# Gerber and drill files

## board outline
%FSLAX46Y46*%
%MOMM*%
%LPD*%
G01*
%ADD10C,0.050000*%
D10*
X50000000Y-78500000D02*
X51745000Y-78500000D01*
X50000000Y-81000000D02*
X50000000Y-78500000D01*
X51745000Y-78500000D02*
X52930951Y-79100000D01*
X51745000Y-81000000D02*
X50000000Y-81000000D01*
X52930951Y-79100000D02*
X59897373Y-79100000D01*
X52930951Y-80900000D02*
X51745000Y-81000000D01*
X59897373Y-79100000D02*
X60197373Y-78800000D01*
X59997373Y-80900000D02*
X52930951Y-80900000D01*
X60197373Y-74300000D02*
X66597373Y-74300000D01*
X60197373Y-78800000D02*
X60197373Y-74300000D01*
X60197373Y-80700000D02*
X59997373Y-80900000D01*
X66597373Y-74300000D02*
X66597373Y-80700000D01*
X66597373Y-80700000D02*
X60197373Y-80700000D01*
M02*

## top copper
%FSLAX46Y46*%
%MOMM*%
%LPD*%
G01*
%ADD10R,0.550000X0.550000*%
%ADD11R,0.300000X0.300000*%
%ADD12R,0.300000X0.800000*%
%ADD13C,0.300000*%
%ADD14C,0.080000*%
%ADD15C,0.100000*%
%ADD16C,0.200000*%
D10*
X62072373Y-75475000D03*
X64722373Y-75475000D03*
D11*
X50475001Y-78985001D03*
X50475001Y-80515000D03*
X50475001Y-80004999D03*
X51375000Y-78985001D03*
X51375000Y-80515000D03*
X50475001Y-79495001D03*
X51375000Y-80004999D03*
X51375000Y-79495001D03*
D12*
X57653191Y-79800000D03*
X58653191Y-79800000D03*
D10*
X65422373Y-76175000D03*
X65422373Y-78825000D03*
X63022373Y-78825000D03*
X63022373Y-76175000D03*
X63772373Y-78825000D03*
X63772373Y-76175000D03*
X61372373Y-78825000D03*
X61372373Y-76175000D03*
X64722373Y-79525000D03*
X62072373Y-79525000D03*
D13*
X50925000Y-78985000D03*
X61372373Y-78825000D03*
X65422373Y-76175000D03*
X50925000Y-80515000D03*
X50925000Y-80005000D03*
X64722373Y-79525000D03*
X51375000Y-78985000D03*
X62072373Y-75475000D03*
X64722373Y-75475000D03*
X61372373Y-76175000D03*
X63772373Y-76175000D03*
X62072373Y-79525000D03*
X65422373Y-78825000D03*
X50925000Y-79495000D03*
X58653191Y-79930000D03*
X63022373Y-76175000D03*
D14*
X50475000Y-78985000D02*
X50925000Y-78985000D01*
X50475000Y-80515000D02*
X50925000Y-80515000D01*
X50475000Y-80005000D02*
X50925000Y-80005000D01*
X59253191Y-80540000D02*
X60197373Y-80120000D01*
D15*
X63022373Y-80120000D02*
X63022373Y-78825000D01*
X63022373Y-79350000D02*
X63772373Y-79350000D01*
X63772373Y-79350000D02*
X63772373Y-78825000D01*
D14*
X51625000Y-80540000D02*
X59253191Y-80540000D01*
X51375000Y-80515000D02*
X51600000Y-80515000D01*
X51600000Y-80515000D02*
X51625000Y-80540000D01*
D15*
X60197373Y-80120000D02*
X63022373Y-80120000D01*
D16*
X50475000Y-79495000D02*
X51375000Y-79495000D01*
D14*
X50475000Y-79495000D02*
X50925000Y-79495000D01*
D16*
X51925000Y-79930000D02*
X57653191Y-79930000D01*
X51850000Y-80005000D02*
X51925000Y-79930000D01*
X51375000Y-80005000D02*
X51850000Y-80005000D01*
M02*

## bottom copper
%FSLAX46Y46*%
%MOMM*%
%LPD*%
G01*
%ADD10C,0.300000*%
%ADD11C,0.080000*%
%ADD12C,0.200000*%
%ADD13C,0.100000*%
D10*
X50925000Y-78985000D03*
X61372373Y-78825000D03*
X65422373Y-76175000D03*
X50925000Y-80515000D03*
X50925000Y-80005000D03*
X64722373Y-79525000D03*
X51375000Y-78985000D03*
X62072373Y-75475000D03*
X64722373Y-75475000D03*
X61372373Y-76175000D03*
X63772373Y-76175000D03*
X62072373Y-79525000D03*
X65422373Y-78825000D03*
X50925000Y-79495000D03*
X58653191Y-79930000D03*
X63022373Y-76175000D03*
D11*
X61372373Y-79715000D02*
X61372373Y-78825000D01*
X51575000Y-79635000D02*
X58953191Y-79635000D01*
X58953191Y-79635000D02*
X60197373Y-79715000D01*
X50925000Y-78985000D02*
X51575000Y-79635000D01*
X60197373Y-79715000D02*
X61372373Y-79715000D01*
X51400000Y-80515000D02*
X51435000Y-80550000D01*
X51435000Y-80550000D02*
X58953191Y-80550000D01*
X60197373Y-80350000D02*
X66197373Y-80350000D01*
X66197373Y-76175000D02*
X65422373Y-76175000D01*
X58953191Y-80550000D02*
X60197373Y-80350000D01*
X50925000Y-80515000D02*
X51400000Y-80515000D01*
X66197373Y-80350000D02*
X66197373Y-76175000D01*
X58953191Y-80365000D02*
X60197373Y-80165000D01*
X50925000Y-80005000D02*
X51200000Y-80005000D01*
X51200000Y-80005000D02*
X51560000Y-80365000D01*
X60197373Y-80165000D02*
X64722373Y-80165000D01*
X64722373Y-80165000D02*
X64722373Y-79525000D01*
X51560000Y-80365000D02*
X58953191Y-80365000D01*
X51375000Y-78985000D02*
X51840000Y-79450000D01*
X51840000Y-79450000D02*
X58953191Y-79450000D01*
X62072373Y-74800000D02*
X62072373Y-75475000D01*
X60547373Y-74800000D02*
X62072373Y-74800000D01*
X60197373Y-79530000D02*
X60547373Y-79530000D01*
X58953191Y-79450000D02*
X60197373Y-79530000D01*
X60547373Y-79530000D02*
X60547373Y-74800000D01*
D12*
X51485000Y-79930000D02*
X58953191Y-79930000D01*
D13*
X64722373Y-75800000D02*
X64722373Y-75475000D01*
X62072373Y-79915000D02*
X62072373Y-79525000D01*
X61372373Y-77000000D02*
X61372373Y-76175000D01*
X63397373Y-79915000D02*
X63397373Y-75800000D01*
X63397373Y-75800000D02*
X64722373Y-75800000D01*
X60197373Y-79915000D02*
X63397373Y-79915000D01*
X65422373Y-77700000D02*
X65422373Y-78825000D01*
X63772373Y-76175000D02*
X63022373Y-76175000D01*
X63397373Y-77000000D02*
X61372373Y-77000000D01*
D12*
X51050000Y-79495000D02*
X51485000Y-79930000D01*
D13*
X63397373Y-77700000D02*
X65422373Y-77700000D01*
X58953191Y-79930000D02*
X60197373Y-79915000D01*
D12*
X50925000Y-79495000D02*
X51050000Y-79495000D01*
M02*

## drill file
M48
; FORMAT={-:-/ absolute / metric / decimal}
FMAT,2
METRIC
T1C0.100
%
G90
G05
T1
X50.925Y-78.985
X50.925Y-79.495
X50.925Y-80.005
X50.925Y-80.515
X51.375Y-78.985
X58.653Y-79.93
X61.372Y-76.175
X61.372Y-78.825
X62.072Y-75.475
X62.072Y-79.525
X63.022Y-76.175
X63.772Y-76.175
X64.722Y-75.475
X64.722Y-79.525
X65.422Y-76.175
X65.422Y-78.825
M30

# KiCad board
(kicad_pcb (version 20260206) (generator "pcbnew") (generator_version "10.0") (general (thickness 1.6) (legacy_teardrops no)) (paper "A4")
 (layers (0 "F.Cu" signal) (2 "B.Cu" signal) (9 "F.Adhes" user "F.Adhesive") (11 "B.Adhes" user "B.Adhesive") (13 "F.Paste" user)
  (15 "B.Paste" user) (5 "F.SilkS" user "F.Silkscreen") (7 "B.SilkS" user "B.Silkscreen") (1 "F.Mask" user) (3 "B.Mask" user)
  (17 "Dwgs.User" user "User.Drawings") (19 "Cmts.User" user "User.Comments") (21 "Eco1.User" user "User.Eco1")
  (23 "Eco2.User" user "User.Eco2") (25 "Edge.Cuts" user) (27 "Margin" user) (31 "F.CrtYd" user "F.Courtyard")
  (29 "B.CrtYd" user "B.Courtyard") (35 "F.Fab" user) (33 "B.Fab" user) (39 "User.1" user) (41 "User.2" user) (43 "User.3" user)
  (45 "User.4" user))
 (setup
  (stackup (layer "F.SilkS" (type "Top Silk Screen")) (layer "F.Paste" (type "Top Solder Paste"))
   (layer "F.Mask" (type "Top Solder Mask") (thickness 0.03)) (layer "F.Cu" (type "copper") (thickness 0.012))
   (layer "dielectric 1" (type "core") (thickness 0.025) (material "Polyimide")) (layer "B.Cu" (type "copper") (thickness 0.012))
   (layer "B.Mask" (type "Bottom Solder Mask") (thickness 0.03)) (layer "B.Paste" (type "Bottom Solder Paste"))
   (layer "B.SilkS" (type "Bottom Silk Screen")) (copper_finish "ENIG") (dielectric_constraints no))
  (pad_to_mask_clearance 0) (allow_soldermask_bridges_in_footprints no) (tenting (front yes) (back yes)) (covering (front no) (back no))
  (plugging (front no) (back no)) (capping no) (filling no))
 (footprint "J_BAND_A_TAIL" (layer "F.Cu") (at 50.9 79.75)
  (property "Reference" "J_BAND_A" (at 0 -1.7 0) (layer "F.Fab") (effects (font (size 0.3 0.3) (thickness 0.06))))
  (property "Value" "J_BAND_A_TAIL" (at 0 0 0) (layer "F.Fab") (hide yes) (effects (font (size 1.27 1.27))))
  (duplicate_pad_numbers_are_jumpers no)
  (pad "1" smd rect (at -0.424999 -0.764999) (size 0.3 0.3) (layers "F.Cu" "F.Mask") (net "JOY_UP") (solder_mask_margin 0.05)
   (thermal_bridge_angle 45))
  (pad "2" smd rect (at -0.424999 0.765) (size 0.3 0.3) (layers "F.Cu" "F.Mask") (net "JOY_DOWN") (solder_mask_margin 0.05)
   (thermal_bridge_angle 45))
  (pad "3" smd rect (at -0.424999 0.254999) (size 0.3 0.3) (layers "F.Cu" "F.Mask") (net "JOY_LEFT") (solder_mask_margin 0.05)
   (thermal_bridge_angle 45))
  (pad "4" smd rect (at 0.475 -0.764999) (size 0.3 0.3) (layers "F.Cu" "F.Mask") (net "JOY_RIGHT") (solder_mask_margin 0.05)
   (thermal_bridge_angle 45))
  (pad "5" smd rect (at 0.475 0.765) (size 0.3 0.3) (layers "F.Cu" "F.Mask") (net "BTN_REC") (solder_mask_margin 0.05)
   (thermal_bridge_angle 45))
  (pad "6" smd rect (at -0.424999 -0.254999) (size 0.3 0.3) (layers "F.Cu" "F.Mask") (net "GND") (solder_mask_margin 0.05)
   (thermal_bridge_angle 45))
  (pad "7" smd rect (at 0.475 0.254999) (size 0.3 0.3) (layers "F.Cu" "F.Mask") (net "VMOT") (solder_mask_margin 0.05)
   (thermal_bridge_angle 45))
  (pad "8" smd rect (at 0.475 -0.254999) (size 0.3 0.3) (layers "F.Cu" "F.Mask") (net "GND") (solder_mask_margin 0.05)
   (thermal_bridge_angle 45)))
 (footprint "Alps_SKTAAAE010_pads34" (layer "F.Cu") (at 60.997373 77.5 90)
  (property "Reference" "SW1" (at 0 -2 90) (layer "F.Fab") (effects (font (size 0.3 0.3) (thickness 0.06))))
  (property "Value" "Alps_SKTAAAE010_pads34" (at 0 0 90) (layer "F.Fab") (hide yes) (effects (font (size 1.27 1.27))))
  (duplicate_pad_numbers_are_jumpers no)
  (pad "3" smd rect (at -1.325 0.375 90) (size 0.55 0.55) (layers "F.Cu" "F.Mask") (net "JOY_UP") (solder_mask_margin 0.05)
   (thermal_bridge_angle 45))
  (pad "4" smd rect (at 1.325 0.375 90) (size 0.55 0.55) (layers "F.Cu" "F.Mask") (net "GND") (solder_mask_margin 0.05)
   (thermal_bridge_angle 45)))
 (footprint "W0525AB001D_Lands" (layer "F.Cu") (at 58.153191 79.93)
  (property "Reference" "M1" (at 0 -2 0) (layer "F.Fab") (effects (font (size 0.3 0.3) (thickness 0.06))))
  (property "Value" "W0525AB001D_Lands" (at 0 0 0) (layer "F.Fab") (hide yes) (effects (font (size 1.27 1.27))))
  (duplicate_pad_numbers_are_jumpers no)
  (pad "1" smd rect (at -0.5 -0.13) (size 0.3 0.8) (layers "F.Cu" "F.Mask") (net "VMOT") (solder_mask_margin 0.05) (thermal_bridge_angle 45))
  (pad "2" smd rect (at 0.5 -0.13) (size 0.3 0.8) (layers "F.Cu" "F.Mask") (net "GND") (solder_mask_margin 0.05) (thermal_bridge_angle 45)))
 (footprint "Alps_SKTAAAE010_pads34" (layer "F.Cu") (at 63.397373 79.9 180)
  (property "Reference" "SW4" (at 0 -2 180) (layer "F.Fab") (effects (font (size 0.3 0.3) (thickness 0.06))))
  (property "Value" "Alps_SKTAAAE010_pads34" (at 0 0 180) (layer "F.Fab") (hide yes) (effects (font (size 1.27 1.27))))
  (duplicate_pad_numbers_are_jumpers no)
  (pad "3" smd rect (at -1.325 0.375 180) (size 0.55 0.55) (layers "F.Cu" "F.Mask") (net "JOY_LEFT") (solder_mask_margin 0.05)
   (thermal_bridge_angle 45))
  (pad "4" smd rect (at 1.325 0.375 180) (size 0.55 0.55) (layers "F.Cu" "F.Mask") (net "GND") (solder_mask_margin 0.05)
   (thermal_bridge_angle 45)))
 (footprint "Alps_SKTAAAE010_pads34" (layer "F.Cu") (at 63.397373 75.1)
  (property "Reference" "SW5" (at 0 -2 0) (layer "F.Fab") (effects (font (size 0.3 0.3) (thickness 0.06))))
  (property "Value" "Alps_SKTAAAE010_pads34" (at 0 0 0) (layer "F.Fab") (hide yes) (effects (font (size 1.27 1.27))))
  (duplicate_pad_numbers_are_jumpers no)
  (pad "3" smd rect (at -1.325 0.375) (size 0.55 0.55) (layers "F.Cu" "F.Mask") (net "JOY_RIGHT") (solder_mask_margin 0.05)
   (thermal_bridge_angle 45))
  (pad "4" smd rect (at 1.325 0.375) (size 0.55 0.55) (layers "F.Cu" "F.Mask") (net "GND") (solder_mask_margin 0.05)
   (thermal_bridge_angle 45)))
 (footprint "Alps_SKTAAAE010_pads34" (layer "F.Cu") (at 65.797373 77.5 -90)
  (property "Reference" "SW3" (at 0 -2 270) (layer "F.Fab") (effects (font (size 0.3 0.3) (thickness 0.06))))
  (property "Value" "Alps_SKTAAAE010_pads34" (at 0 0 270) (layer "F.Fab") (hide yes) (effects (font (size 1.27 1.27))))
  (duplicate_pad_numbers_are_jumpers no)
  (pad "3" smd rect (at -1.325 0.375 270) (size 0.55 0.55) (layers "F.Cu" "F.Mask") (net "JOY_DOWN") (solder_mask_margin 0.05)
   (thermal_bridge_angle 45))
  (pad "4" smd rect (at 1.325 0.375 270) (size 0.55 0.55) (layers "F.Cu" "F.Mask") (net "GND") (solder_mask_margin 0.05)
   (thermal_bridge_angle 45)))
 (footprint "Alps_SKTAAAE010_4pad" (layer "F.Cu") (at 63.397373 77.5 90)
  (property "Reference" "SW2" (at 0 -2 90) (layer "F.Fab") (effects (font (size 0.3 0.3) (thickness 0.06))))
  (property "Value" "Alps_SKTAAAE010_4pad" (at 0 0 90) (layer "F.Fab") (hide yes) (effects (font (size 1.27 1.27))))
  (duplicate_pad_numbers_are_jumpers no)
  (pad "1" smd rect (at -1.325 -0.375 90) (size 0.55 0.55) (layers "F.Cu" "F.Mask") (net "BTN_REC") (solder_mask_margin 0.05)
   (thermal_bridge_angle 45))
  (pad "2" smd rect (at 1.325 -0.375 90) (size 0.55 0.55) (layers "F.Cu" "F.Mask") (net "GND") (solder_mask_margin 0.05)
   (thermal_bridge_angle 45))
  (pad "3" smd rect (at -1.325 0.375 90) (size 0.55 0.55) (layers "F.Cu" "F.Mask") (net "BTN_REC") (solder_mask_margin 0.05)
   (thermal_bridge_angle 45))
  (pad "4" smd rect (at 1.325 0.375 90) (size 0.55 0.55) (layers "F.Cu" "F.Mask") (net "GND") (solder_mask_margin 0.05)
   (thermal_bridge_angle 45)))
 (gr_line (start 50 78.5) (end 51.745 78.5) (stroke (width 0.05) (type default)) (layer "Edge.Cuts"))
 (gr_line (start 50 81) (end 50 78.5) (stroke (width 0.05) (type default)) (layer "Edge.Cuts"))
 (gr_line (start 51.745 78.5) (end 52.930951 79.1) (stroke (width 0.05) (type default)) (layer "Edge.Cuts"))
 (gr_line (start 51.745 81) (end 50 81) (stroke (width 0.05) (type default)) (layer "Edge.Cuts"))
 (gr_line (start 52.930951 79.1) (end 59.897373 79.1) (stroke (width 0.05) (type default)) (layer "Edge.Cuts"))
 (gr_line (start 52.930951 80.9) (end 51.745 81) (stroke (width 0.05) (type default)) (layer "Edge.Cuts"))
 (gr_line (start 59.897373 79.1) (end 60.197373 78.8) (stroke (width 0.05) (type default)) (layer "Edge.Cuts"))
 (gr_line (start 59.997373 80.9) (end 52.930951 80.9) (stroke (width 0.05) (type default)) (layer "Edge.Cuts"))
 (gr_line (start 60.197373 74.3) (end 66.597373 74.3) (stroke (width 0.05) (type default)) (layer "Edge.Cuts"))
 (gr_line (start 60.197373 78.8) (end 60.197373 74.3) (stroke (width 0.05) (type default)) (layer "Edge.Cuts"))
 (gr_line (start 60.197373 80.7) (end 59.997373 80.9) (stroke (width 0.05) (type default)) (layer "Edge.Cuts"))
 (gr_line (start 66.597373 74.3) (end 66.597373 80.7) (stroke (width 0.05) (type default)) (layer "Edge.Cuts"))
 (gr_line (start 66.597373 80.7) (end 60.197373 80.7) (stroke (width 0.05) (type default)) (layer "Edge.Cuts"))
 (segment (start 50.475 78.985) (end 50.925 78.985) (width 0.08) (layer "F.Cu") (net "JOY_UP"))
 (via (at 61.372373 78.825) (size 0.3) (drill 0.1) (layers "F.Cu" "B.Cu") (tenting (front yes) (back yes)) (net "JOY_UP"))
 (via (at 50.925 78.985) (size 0.3) (drill 0.1) (layers "F.Cu" "B.Cu") (tenting (front yes) (back yes)) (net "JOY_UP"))
 (segment (start 58.953191 79.635) (end 60.197373 79.715) (width 0.08) (layer "B.Cu") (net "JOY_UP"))
 (segment (start 60.197373 79.715) (end 61.372373 79.715) (width 0.08) (layer "B.Cu") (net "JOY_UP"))
 (segment (start 61.372373 79.715) (end 61.372373 78.825) (width 0.08) (layer "B.Cu") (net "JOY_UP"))
 (segment (start 50.925 78.985) (end 51.575 79.635) (width 0.08) (layer "B.Cu") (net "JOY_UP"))
 (segment (start 51.575 79.635) (end 58.953191 79.635) (width 0.08) (layer "B.Cu") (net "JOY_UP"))
 (segment (start 50.475 80.515) (end 50.925 80.515) (width 0.08) (layer "F.Cu") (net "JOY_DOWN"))
 (via (at 65.422373 76.175) (size 0.3) (drill 0.1) (layers "F.Cu" "B.Cu") (tenting (front yes) (back yes)) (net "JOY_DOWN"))
 (via (at 50.925 80.515) (size 0.3) (drill 0.1) (layers "F.Cu" "B.Cu") (tenting (front yes) (back yes)) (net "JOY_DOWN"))
 (segment (start 50.925 80.515) (end 51.4 80.515) (width 0.08) (layer "B.Cu") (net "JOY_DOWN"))
 (segment (start 66.197373 80.35) (end 66.197373 76.175) (width 0.08) (layer "B.Cu") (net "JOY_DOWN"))
 (segment (start 51.435 80.55) (end 58.953191 80.55) (width 0.08) (layer "B.Cu") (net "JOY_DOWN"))
 (segment (start 58.953191 80.55) (end 60.197373 80.35) (width 0.08) (layer "B.Cu") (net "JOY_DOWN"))
 (segment (start 51.4 80.515) (end 51.435 80.55) (width 0.08) (layer "B.Cu") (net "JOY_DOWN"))
 (segment (start 66.197373 76.175) (end 65.422373 76.175) (width 0.08) (layer "B.Cu") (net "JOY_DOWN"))
 (segment (start 60.197373 80.35) (end 66.197373 80.35) (width 0.08) (layer "B.Cu") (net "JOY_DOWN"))
 (segment (start 50.475 80.005) (end 50.925 80.005) (width 0.08) (layer "F.Cu") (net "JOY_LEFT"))
 (via (at 64.722373 79.525) (size 0.3) (drill 0.1) (layers "F.Cu" "B.Cu") (tenting (front yes) (back yes)) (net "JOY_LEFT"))
 (via (at 50.925 80.005) (size 0.3) (drill 0.1) (layers "F.Cu" "B.Cu") (tenting (front yes) (back yes)) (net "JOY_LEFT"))
 (segment (start 58.953191 80.365) (end 60.197373 80.165) (width 0.08) (layer "B.Cu") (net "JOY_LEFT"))
 (segment (start 51.2 80.005) (end 51.56 80.365) (width 0.08) (layer "B.Cu") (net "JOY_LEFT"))
 (segment (start 60.197373 80.165) (end 64.722373 80.165) (width 0.08) (layer "B.Cu") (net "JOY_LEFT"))
 (segment (start 64.722373 80.165) (end 64.722373 79.525) (width 0.08) (layer "B.Cu") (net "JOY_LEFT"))
 (segment (start 50.925 80.005) (end 51.2 80.005) (width 0.08) (layer "B.Cu") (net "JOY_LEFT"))
 (segment (start 51.56 80.365) (end 58.953191 80.365) (width 0.08) (layer "B.Cu") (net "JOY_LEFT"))
 (via (at 62.072373 75.475) (size 0.3) (drill 0.1) (layers "F.Cu" "B.Cu") (tenting (front yes) (back yes)) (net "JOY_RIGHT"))
 (via (at 51.375 78.985) (size 0.3) (drill 0.1) (layers "F.Cu" "B.Cu") (tenting (front yes) (back yes)) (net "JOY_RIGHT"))
 (segment (start 60.197373 79.53) (end 60.547373 79.53) (width 0.08) (layer "B.Cu") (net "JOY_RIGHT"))
 (segment (start 58.953191 79.45) (end 60.197373 79.53) (width 0.08) (layer "B.Cu") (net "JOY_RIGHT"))
 (segment (start 51.375 78.985) (end 51.84 79.45) (width 0.08) (layer "B.Cu") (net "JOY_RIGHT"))
 (segment (start 60.547373 79.53) (end 60.547373 74.8) (width 0.08) (layer "B.Cu") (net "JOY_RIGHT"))
 (segment (start 62.072373 74.8) (end 62.072373 75.475) (width 0.08) (layer "B.Cu") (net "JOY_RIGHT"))
 (segment (start 60.547373 74.8) (end 62.072373 74.8) (width 0.08) (layer "B.Cu") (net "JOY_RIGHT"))
 (segment (start 51.84 79.45) (end 58.953191 79.45) (width 0.08) (layer "B.Cu") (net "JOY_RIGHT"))
 (segment (start 63.022373 79.35) (end 63.772373 79.35) (width 0.1) (layer "F.Cu") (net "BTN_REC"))
 (segment (start 51.375 80.515) (end 51.6 80.515) (width 0.08) (layer "F.Cu") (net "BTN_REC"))
 (segment (start 60.197373 80.12) (end 63.022373 80.12) (width 0.1) (layer "F.Cu") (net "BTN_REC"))
 (segment (start 59.253191 80.54) (end 60.197373 80.12) (width 0.08) (layer "F.Cu") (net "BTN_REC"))
 (segment (start 63.772373 79.35) (end 63.772373 78.825) (width 0.1) (layer "F.Cu") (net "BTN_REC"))
 (segment (start 51.625 80.54) (end 59.253191 80.54) (width 0.08) (layer "F.Cu") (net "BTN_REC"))
 (segment (start 51.6 80.515) (end 51.625 80.54) (width 0.08) (layer "F.Cu") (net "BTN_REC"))
 (segment (start 63.022373 80.12) (end 63.022373 78.825) (width 0.1) (layer "F.Cu") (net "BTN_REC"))
 (segment (start 50.475 79.495) (end 51.375 79.495) (width 0.2) (layer "F.Cu") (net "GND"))
 (segment (start 50.475 79.495) (end 50.925 79.495) (width 0.08) (layer "F.Cu") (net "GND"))
 (via (at 50.925 79.495) (size 0.3) (drill 0.1) (layers "F.Cu" "B.Cu") (tenting (front yes) (back yes)) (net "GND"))
 (via (at 63.022373 76.175) (size 0.3) (drill 0.1) (layers "F.Cu" "B.Cu") (tenting (front yes) (back yes)) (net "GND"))
 (via (at 63.772373 76.175) (size 0.3) (drill 0.1) (layers "F.Cu" "B.Cu") (tenting (front yes) (back yes)) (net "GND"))
 (via (at 61.372373 76.175) (size 0.3) (drill 0.1) (layers "F.Cu" "B.Cu") (tenting (front yes) (back yes)) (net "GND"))
 (via (at 58.653191 79.93) (size 0.3) (drill 0.1) (layers "F.Cu" "B.Cu") (tenting (front yes) (back yes)) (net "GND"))
 (via (at 62.072373 79.525) (size 0.3) (drill 0.1) (layers "F.Cu" "B.Cu") (tenting (front yes) (back yes)) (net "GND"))
 (via (at 64.722373 75.475) (size 0.3) (drill 0.1) (layers "F.Cu" "B.Cu") (tenting (front yes) (back yes)) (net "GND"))
 (via (at 65.422373 78.825) (size 0.3) (drill 0.1) (layers "F.Cu" "B.Cu") (tenting (front yes) (back yes)) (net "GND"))
 (segment (start 64.722373 75.8) (end 64.722373 75.475) (width 0.1) (layer "B.Cu") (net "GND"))
 (segment (start 63.772373 76.175) (end 63.022373 76.175) (width 0.1) (layer "B.Cu") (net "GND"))
 (segment (start 61.372373 77) (end 61.372373 76.175) (width 0.1) (layer "B.Cu") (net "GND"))
 (segment (start 62.072373 79.915) (end 62.072373 79.525) (width 0.1) (layer "B.Cu") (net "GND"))
 (segment (start 63.397373 79.915) (end 63.397373 75.8) (width 0.1) (layer "B.Cu") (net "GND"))
 (segment (start 50.925 79.495) (end 51.05 79.495) (width 0.2) (layer "B.Cu") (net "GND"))
 (segment (start 63.397373 75.8) (end 64.722373 75.8) (width 0.1) (layer "B.Cu") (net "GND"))
 (segment (start 65.422373 77.7) (end 65.422373 78.825) (width 0.1) (layer "B.Cu") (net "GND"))
 (segment (start 51.05 79.495) (end 51.485 79.93) (width 0.2) (layer "B.Cu") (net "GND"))
 (segment (start 63.397373 77.7) (end 65.422373 77.7) (width 0.1) (layer "B.Cu") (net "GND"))
 (segment (start 58.953191 79.93) (end 60.197373 79.915) (width 0.1) (layer "B.Cu") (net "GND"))
 (segment (start 60.197373 79.915) (end 63.397373 79.915) (width 0.1) (layer "B.Cu") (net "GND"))
 (segment (start 51.485 79.93) (end 58.953191 79.93) (width 0.2) (layer "B.Cu") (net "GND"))
 (segment (start 63.397373 77) (end 61.372373 77) (width 0.1) (layer "B.Cu") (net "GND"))
 (segment (start 51.85 80.005) (end 51.925 79.93) (width 0.2) (layer "F.Cu") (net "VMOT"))
 (segment (start 51.375 80.005) (end 51.85 80.005) (width 0.2) (layer "F.Cu") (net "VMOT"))
 (segment (start 51.925 79.93) (end 57.653191 79.93) (width 0.2) (layer "F.Cu") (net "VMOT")))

